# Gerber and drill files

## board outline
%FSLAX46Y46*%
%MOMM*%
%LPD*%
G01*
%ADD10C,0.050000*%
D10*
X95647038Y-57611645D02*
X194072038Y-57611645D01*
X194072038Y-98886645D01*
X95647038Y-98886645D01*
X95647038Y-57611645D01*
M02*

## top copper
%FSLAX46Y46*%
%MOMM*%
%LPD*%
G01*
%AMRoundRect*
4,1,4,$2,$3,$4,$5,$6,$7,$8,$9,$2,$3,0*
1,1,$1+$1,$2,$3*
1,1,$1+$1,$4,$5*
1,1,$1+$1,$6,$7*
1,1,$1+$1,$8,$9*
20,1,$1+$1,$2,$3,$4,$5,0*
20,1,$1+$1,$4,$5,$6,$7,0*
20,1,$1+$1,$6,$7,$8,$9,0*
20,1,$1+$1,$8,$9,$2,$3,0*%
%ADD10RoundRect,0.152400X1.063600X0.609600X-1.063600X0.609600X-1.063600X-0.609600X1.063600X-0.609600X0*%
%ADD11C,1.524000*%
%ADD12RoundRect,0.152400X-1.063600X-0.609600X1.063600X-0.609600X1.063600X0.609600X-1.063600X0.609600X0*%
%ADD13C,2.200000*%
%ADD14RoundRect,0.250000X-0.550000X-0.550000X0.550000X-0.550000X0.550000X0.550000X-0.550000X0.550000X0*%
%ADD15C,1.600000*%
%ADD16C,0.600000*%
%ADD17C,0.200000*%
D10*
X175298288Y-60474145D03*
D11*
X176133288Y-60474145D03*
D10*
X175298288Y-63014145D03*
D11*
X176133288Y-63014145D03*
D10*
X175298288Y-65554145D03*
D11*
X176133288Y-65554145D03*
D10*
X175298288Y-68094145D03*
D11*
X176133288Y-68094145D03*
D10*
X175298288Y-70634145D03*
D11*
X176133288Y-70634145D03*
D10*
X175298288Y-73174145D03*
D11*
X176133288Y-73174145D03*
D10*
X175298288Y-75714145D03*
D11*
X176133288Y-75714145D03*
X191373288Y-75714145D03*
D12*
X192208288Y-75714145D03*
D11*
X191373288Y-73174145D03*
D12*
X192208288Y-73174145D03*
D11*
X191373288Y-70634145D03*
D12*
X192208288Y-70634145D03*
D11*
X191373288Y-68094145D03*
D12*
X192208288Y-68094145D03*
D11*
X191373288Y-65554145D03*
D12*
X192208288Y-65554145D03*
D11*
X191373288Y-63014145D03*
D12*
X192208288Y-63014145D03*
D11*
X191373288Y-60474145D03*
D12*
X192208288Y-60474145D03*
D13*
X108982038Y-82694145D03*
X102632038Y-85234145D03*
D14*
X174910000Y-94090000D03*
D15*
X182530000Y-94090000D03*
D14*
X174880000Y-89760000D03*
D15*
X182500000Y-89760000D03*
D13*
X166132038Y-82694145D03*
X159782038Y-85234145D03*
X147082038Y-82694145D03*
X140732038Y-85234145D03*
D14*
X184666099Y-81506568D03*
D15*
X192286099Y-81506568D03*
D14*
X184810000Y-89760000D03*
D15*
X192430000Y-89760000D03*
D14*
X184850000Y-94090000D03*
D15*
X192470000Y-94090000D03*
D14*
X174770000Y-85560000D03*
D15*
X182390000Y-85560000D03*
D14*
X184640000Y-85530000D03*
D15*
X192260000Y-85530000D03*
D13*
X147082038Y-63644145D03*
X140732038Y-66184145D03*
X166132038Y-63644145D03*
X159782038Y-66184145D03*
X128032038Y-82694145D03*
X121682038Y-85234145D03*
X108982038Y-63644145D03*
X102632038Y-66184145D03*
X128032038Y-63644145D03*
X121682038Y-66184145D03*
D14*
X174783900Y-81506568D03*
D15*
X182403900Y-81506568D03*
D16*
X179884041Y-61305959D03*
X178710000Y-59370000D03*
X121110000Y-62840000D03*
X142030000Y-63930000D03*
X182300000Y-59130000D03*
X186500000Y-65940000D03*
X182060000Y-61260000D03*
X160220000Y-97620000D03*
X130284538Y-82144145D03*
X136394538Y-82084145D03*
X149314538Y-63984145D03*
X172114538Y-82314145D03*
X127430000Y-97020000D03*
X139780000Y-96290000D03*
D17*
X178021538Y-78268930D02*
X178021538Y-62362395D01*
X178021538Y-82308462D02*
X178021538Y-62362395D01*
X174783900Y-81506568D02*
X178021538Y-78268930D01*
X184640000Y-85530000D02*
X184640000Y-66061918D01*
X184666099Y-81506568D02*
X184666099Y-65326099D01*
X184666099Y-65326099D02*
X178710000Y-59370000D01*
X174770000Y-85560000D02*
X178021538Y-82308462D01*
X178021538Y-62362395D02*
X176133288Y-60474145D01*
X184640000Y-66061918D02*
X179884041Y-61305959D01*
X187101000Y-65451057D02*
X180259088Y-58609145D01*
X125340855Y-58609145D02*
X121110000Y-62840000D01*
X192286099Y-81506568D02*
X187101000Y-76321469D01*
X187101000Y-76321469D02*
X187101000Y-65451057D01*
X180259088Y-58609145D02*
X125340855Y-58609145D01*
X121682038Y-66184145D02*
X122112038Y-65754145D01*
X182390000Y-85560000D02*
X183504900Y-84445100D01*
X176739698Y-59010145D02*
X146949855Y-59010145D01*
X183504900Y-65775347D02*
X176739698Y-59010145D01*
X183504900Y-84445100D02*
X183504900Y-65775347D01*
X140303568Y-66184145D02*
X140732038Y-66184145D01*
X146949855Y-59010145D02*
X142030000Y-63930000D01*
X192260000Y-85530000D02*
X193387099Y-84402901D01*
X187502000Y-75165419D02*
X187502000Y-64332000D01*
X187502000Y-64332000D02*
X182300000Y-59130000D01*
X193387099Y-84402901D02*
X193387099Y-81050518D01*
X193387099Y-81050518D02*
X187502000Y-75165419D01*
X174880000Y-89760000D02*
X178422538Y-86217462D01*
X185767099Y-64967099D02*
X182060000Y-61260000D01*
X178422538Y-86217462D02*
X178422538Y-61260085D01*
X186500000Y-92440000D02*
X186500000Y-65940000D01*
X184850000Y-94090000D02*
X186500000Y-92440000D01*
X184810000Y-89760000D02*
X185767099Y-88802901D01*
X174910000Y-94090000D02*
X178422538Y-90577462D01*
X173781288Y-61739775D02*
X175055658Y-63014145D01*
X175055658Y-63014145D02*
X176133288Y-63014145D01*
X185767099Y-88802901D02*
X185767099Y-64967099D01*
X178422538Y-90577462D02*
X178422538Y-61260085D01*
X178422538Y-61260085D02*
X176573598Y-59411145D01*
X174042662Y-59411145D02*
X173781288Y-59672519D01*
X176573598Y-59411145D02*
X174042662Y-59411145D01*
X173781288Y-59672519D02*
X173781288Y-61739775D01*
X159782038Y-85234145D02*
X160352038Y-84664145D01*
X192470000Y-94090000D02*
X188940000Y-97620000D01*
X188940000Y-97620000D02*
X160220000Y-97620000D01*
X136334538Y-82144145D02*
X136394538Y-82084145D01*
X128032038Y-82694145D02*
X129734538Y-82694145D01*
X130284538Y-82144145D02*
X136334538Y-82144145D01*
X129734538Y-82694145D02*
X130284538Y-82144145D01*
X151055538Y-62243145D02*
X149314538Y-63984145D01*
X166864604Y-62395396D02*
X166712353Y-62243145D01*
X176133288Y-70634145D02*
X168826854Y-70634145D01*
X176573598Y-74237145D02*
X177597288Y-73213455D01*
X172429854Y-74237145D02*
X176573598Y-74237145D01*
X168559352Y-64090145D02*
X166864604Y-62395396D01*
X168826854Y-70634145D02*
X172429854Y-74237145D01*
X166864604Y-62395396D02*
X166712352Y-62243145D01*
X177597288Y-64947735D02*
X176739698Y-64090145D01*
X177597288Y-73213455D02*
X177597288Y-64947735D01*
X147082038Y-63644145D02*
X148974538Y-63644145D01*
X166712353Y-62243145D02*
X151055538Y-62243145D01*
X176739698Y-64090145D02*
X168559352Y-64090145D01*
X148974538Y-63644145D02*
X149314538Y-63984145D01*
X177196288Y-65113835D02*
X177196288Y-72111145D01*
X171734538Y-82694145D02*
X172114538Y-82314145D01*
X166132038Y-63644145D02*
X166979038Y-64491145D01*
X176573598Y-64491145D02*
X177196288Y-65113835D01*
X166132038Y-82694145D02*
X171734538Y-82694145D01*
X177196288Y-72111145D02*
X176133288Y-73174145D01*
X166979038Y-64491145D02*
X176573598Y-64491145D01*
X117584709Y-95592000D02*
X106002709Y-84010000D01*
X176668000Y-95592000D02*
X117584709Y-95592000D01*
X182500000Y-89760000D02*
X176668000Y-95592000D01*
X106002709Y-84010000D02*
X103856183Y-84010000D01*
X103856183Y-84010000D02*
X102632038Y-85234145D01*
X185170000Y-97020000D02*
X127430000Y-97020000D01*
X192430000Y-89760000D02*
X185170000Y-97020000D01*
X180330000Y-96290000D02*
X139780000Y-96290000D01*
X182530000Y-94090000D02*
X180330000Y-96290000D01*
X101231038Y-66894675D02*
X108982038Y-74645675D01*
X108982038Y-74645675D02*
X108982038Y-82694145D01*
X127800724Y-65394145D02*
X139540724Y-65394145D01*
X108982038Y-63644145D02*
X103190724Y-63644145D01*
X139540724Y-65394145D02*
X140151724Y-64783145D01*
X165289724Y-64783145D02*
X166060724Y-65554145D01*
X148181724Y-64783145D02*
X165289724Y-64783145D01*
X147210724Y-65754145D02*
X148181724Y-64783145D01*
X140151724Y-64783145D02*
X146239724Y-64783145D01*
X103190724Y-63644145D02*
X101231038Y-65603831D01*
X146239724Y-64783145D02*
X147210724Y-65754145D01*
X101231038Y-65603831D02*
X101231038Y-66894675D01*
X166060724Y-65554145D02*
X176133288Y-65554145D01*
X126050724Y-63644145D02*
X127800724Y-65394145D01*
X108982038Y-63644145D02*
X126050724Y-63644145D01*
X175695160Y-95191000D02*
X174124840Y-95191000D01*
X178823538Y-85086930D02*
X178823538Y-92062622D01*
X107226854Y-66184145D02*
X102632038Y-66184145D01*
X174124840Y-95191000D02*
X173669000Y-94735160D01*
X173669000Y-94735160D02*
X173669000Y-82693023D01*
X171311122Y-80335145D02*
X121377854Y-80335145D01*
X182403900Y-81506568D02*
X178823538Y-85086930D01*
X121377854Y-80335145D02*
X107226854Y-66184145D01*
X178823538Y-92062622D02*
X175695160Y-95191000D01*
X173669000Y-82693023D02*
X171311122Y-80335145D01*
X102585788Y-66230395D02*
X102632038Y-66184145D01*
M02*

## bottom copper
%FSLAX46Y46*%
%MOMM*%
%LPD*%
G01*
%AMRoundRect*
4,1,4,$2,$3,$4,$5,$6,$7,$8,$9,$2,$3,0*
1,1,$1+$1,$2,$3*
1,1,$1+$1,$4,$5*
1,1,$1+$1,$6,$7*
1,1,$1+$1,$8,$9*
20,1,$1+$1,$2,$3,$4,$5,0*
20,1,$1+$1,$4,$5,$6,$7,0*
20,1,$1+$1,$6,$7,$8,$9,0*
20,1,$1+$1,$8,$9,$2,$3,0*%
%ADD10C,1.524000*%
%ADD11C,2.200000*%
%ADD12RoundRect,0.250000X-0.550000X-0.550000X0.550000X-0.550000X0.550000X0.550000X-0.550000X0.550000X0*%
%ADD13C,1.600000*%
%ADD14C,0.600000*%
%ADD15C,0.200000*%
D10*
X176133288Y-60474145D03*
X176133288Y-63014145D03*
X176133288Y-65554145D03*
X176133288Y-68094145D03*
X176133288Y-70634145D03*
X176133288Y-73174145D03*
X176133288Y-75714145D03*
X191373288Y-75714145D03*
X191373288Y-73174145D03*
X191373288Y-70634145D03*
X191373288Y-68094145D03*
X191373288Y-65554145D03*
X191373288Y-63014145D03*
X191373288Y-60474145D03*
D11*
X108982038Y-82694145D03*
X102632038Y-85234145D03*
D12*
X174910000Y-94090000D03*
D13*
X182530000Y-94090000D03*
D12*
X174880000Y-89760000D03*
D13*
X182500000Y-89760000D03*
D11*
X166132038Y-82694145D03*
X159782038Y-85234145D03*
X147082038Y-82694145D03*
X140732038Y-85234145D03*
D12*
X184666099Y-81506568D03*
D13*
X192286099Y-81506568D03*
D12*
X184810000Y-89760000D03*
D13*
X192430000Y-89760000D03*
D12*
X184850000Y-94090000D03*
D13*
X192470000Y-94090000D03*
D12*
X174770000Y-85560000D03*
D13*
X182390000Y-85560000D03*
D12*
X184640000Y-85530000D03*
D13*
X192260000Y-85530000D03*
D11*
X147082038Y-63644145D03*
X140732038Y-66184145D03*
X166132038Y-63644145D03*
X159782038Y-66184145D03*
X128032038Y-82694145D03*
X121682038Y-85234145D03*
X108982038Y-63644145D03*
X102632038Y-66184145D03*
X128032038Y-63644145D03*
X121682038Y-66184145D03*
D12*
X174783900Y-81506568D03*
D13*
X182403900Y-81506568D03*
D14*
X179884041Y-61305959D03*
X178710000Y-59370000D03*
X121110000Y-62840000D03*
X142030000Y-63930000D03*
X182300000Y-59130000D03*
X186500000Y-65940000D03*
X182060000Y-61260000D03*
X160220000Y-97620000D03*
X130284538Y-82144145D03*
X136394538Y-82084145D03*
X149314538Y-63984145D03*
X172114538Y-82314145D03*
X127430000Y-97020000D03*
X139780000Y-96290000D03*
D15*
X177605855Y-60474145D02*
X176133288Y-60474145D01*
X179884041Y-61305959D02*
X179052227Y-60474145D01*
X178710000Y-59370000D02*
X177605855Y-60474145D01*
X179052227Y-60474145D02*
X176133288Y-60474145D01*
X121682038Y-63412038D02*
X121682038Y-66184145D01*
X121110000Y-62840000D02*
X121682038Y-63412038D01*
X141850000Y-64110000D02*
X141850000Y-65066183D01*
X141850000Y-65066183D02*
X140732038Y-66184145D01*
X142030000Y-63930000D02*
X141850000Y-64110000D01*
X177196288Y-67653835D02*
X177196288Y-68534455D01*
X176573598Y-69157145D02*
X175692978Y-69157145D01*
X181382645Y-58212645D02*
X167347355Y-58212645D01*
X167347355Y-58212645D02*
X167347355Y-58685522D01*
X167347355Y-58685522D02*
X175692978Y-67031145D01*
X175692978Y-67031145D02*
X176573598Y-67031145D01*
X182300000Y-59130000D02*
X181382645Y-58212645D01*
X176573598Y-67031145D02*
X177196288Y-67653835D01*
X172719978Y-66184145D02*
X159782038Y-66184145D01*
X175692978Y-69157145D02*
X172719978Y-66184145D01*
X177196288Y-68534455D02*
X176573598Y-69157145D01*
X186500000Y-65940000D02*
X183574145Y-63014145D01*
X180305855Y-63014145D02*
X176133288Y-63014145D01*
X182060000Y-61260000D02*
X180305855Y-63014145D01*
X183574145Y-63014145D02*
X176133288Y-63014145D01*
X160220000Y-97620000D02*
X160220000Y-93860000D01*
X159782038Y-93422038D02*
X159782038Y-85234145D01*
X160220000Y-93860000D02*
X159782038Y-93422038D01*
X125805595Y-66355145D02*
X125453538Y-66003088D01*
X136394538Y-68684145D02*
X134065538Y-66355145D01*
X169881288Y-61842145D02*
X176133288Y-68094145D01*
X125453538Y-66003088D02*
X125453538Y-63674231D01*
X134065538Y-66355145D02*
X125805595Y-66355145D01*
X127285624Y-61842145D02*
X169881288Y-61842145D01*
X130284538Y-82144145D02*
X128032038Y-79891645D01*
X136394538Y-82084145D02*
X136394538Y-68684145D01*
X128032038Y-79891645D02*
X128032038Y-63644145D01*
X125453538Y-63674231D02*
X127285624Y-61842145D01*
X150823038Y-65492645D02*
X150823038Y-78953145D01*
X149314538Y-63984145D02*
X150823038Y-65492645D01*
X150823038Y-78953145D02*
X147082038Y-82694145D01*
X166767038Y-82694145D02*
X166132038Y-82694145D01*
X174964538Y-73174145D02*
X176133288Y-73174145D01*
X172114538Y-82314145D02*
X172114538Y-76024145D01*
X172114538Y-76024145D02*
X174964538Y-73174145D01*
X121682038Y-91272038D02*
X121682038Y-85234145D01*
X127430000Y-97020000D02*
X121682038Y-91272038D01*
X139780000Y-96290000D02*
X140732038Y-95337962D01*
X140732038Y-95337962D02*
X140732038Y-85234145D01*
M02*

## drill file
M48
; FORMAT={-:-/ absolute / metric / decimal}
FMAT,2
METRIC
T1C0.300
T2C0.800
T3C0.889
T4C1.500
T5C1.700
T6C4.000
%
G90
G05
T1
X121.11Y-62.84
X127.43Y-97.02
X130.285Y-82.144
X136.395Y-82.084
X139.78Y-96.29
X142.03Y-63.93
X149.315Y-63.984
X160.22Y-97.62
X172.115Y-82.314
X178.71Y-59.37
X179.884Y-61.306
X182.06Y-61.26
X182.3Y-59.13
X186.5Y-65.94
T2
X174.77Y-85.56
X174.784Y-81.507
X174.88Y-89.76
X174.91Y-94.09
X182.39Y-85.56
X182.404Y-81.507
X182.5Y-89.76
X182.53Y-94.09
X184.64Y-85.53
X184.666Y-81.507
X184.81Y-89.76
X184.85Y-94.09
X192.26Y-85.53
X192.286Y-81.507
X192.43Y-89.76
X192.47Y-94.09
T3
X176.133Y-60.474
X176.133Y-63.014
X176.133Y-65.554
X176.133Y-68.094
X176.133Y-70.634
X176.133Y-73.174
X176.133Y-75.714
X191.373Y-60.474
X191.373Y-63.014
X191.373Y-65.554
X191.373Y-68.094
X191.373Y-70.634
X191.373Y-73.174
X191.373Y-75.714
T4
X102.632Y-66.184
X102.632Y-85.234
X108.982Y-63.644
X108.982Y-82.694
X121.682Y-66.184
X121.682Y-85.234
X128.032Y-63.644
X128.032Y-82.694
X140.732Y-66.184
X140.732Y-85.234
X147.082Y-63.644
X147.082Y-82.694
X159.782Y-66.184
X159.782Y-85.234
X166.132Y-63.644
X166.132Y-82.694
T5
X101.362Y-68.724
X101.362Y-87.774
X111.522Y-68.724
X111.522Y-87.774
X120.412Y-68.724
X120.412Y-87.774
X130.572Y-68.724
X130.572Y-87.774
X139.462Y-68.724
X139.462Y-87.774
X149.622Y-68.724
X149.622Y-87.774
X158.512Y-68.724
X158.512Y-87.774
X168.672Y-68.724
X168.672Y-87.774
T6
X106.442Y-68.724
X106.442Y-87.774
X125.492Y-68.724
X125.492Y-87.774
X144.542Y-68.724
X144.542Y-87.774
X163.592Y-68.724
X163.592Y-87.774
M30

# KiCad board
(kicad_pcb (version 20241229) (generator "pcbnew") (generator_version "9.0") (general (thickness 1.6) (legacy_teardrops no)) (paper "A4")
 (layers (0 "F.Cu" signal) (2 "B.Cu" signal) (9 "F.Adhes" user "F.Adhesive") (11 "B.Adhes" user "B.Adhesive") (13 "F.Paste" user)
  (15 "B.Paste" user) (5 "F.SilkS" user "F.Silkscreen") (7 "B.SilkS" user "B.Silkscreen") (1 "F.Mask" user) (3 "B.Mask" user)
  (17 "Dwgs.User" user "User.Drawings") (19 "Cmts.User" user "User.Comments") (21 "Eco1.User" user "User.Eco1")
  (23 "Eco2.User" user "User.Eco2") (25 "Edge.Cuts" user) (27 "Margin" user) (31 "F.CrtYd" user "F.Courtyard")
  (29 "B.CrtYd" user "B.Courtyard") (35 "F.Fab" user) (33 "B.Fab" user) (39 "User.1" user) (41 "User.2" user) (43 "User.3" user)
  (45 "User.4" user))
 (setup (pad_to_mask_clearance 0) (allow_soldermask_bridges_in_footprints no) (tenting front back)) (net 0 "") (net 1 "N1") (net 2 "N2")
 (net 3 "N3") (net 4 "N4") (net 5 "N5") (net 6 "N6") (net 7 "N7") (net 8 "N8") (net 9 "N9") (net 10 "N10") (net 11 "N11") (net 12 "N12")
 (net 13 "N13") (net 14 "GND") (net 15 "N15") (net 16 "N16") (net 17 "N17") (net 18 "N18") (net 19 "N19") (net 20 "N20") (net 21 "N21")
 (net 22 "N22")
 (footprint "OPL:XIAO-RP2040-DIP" (layer "F.Cu") (at 183.753288 68.094145)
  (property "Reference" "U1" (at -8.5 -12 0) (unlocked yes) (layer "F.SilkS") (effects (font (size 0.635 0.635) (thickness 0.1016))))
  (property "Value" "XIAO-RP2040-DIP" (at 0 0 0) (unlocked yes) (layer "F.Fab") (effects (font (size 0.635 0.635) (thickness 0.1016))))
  (pad "1" smd roundrect (at -8.455 -7.62 180) (size 2.432 1.524) (layers "F.Cu" "F.Mask") (roundrect_rratio 0.1) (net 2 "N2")
   (thermal_bridge_angle 45))
  (pad "1" thru_hole circle (at -7.62 -7.62 180) (size 1.524 1.524) (drill 0.889) (layers "*.Cu" "*.Mask") (remove_unused_layers no)
   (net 2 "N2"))
  (pad "2" smd roundrect (at -8.455 -5.08 180) (size 2.432 1.524) (layers "F.Cu" "F.Mask") (roundrect_rratio 0.1) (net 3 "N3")
   (thermal_bridge_angle 45))
  (pad "2" thru_hole circle (at -7.62 -5.08 180) (size 1.524 1.524) (drill 0.889) (layers "*.Cu" "*.Mask") (remove_unused_layers no)
   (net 3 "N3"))
  (pad "3" smd roundrect (at -8.455 -2.54 180) (size 2.432 1.524) (layers "F.Cu" "F.Mask") (roundrect_rratio 0.1) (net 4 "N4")
   (thermal_bridge_angle 45))
  (pad "3" thru_hole circle (at -7.62 -2.54 180) (size 1.524 1.524) (drill 0.889) (layers "*.Cu" "*.Mask") (remove_unused_layers no)
   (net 4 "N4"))
  (pad "4" smd roundrect (at -8.455 0 180) (size 2.432 1.524) (layers "F.Cu" "F.Mask") (roundrect_rratio 0.1) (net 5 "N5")
   (thermal_bridge_angle 45))
  (pad "4" thru_hole circle (at -7.62 0 180) (size 1.524 1.524) (drill 0.889) (layers "*.Cu" "*.Mask") (remove_unused_layers no)
   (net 5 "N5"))
  (pad "5" smd roundrect (at -8.455 2.54 180) (size 2.432 1.524) (layers "F.Cu" "F.Mask") (roundrect_rratio 0.1) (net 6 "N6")
   (thermal_bridge_angle 45))
  (pad "5" thru_hole circle (at -7.62 2.54 180) (size 1.524 1.524) (drill 0.889) (layers "*.Cu" "*.Mask") (remove_unused_layers no)
   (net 6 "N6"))
  (pad "6" smd roundrect (at -8.455 5.08 180) (size 2.432 1.524) (layers "F.Cu" "F.Mask") (roundrect_rratio 0.1) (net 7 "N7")
   (thermal_bridge_angle 45))
  (pad "6" thru_hole circle (at -7.62 5.08 180) (size 1.524 1.524) (drill 0.889) (layers "*.Cu" "*.Mask") (remove_unused_layers no)
   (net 7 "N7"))
  (pad "7" smd roundrect (at -8.455 7.62 180) (size 2.432 1.524) (layers "F.Cu" "F.Mask") (roundrect_rratio 0.1) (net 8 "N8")
   (thermal_bridge_angle 45))
  (pad "7" thru_hole circle (at -7.62 7.62 180) (size 1.524 1.524) (drill 0.889) (layers "*.Cu" "*.Mask") (remove_unused_layers no)
   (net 8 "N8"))
  (pad "8" thru_hole circle (at 7.62 7.62) (size 1.524 1.524) (drill 0.889) (layers "*.Cu" "*.Mask") (remove_unused_layers no) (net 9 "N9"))
  (pad "8" smd roundrect (at 8.455 7.62) (size 2.432 1.524) (layers "F.Cu" "F.Mask") (roundrect_rratio 0.1) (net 9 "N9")
   (thermal_bridge_angle 45))
  (pad "9" thru_hole circle (at 7.62 5.08) (size 1.524 1.524) (drill 0.889) (layers "*.Cu" "*.Mask") (remove_unused_layers no)
   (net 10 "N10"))
  (pad "9" smd roundrect (at 8.455 5.08) (size 2.432 1.524) (layers "F.Cu" "F.Mask") (roundrect_rratio 0.1) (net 10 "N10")
   (thermal_bridge_angle 45))
  (pad "10" thru_hole circle (at 7.62 2.54) (size 1.524 1.524) (drill 0.889) (layers "*.Cu" "*.Mask") (remove_unused_layers no)
   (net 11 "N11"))
  (pad "10" smd roundrect (at 8.455 2.54) (size 2.432 1.524) (layers "F.Cu" "F.Mask") (roundrect_rratio 0.1) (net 11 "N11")
   (thermal_bridge_angle 45))
  (pad "11" thru_hole circle (at 7.62 0) (size 1.524 1.524) (drill 0.889) (layers "*.Cu" "*.Mask") (remove_unused_layers no) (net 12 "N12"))
  (pad "11" smd roundrect (at 8.455 0) (size 2.432 1.524) (layers "F.Cu" "F.Mask") (roundrect_rratio 0.1) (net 12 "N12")
   (thermal_bridge_angle 45))
  (pad "12" thru_hole circle (at 7.62 -2.54) (size 1.524 1.524) (drill 0.889) (layers "*.Cu" "*.Mask") (remove_unused_layers no)
   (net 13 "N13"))
  (pad "12" smd roundrect (at 8.455 -2.54) (size 2.432 1.524) (layers "F.Cu" "F.Mask") (roundrect_rratio 0.1) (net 13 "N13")
   (thermal_bridge_angle 45))
  (pad "13" thru_hole circle (at 7.62 -5.08) (size 1.524 1.524) (drill 0.889) (layers "*.Cu" "*.Mask") (remove_unused_layers no)
   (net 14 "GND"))
  (pad "13" smd roundrect (at 8.455 -5.08) (size 2.432 1.524) (layers "F.Cu" "F.Mask") (roundrect_rratio 0.1) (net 14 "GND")
   (thermal_bridge_angle 45))
  (pad "14" thru_hole circle (at 7.62 -7.62) (size 1.524 1.524) (drill 0.889) (layers "*.Cu" "*.Mask") (remove_unused_layers no)
   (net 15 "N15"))
  (pad "14" smd roundrect (at 8.455 -7.62) (size 2.432 1.524) (layers "F.Cu" "F.Mask") (roundrect_rratio 0.1) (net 15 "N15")
   (thermal_bridge_angle 45)))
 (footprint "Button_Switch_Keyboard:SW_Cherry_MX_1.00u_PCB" (layer "F.Cu") (at 108.982038 82.694145)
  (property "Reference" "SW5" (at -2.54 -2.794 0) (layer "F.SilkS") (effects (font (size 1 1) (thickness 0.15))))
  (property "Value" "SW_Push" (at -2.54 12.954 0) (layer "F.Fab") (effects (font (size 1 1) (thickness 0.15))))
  (pad "" np_thru_hole circle (at -7.62 5.08) (size 1.7 1.7) (drill 1.7) (layers "*.Cu" "*.Mask"))
  (pad "" np_thru_hole circle (at -2.54 5.08) (size 4 4) (drill 4) (layers "*.Cu" "*.Mask"))
  (pad "" np_thru_hole circle (at 2.54 5.08) (size 1.7 1.7) (drill 1.7) (layers "*.Cu" "*.Mask"))
  (pad "1" thru_hole circle (at 0 0) (size 2.2 2.2) (drill 1.5) (layers "*.Cu" "*.Mask") (remove_unused_layers no) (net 4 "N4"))
  (pad "2" thru_hole circle (at -6.35 2.54) (size 2.2 2.2) (drill 1.5) (layers "*.Cu" "*.Mask") (remove_unused_layers no) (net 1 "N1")))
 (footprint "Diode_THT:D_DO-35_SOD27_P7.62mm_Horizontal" (layer "F.Cu") (at 174.91 94.09)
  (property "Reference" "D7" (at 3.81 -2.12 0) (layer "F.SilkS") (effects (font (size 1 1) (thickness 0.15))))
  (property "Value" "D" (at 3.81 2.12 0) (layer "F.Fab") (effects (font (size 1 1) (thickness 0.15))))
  (pad "1" thru_hole roundrect (at 0 0) (size 1.6 1.6) (drill 0.8) (layers "*.Cu" "*.Mask") (remove_unused_layers no)
   (roundrect_rratio 0.15625) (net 3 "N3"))
  (pad "2" thru_hole circle (at 7.62 0) (size 1.6 1.6) (drill 0.8) (layers "*.Cu" "*.Mask") (remove_unused_layers no) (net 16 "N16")))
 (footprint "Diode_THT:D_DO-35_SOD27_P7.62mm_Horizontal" (layer "F.Cu") (at 174.88 89.76)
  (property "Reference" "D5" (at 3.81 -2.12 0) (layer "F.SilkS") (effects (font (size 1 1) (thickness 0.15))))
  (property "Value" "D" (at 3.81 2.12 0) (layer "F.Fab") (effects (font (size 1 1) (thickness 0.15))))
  (pad "1" thru_hole roundrect (at 0 0) (size 1.6 1.6) (drill 0.8) (layers "*.Cu" "*.Mask") (remove_unused_layers no)
   (roundrect_rratio 0.15625) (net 3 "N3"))
  (pad "2" thru_hole circle (at 7.62 0) (size 1.6 1.6) (drill 0.8) (layers "*.Cu" "*.Mask") (remove_unused_layers no) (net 1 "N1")))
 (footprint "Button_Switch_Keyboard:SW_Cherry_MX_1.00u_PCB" (layer "F.Cu") (at 166.132038 82.694145)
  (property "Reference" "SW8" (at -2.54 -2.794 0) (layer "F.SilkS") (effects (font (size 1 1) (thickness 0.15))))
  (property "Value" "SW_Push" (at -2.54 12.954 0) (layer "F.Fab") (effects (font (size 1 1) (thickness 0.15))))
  (pad "" np_thru_hole circle (at -7.62 5.08) (size 1.7 1.7) (drill 1.7) (layers "*.Cu" "*.Mask"))
  (pad "" np_thru_hole circle (at -2.54 5.08) (size 4 4) (drill 4) (layers "*.Cu" "*.Mask"))
  (pad "" np_thru_hole circle (at 2.54 5.08) (size 1.7 1.7) (drill 1.7) (layers "*.Cu" "*.Mask"))
  (pad "1" thru_hole circle (at 0 0) (size 2.2 2.2) (drill 1.5) (layers "*.Cu" "*.Mask") (remove_unused_layers no) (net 7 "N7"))
  (pad "2" thru_hole circle (at -6.35 2.54) (size 2.2 2.2) (drill 1.5) (layers "*.Cu" "*.Mask") (remove_unused_layers no) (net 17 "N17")))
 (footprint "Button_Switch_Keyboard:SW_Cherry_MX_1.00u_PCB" (layer "F.Cu") (at 147.082038 82.694145)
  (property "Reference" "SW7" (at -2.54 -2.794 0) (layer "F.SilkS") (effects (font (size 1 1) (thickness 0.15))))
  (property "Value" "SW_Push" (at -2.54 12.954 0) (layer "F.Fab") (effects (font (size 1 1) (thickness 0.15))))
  (pad "" np_thru_hole circle (at -7.62 5.08) (size 1.7 1.7) (drill 1.7) (layers "*.Cu" "*.Mask"))
  (pad "" np_thru_hole circle (at -2.54 5.08) (size 4 4) (drill 4) (layers "*.Cu" "*.Mask"))
  (pad "" np_thru_hole circle (at 2.54 5.08) (size 1.7 1.7) (drill 1.7) (layers "*.Cu" "*.Mask"))
  (pad "1" thru_hole circle (at 0 0) (size 2.2 2.2) (drill 1.5) (layers "*.Cu" "*.Mask") (remove_unused_layers no) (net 6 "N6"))
  (pad "2" thru_hole circle (at -6.35 2.54) (size 2.2 2.2) (drill 1.5) (layers "*.Cu" "*.Mask") (remove_unused_layers no) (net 16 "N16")))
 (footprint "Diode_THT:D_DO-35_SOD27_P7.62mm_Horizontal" (layer "F.Cu") (at 184.666099 81.506568)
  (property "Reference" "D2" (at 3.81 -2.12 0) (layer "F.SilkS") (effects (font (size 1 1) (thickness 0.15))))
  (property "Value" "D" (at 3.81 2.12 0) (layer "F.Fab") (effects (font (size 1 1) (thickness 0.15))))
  (pad "1" thru_hole roundrect (at 0 0) (size 1.6 1.6) (drill 0.8) (layers "*.Cu" "*.Mask") (remove_unused_layers no)
   (roundrect_rratio 0.15625) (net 2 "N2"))
  (pad "2" thru_hole circle (at 7.62 0) (size 1.6 1.6) (drill 0.8) (layers "*.Cu" "*.Mask") (remove_unused_layers no) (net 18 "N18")))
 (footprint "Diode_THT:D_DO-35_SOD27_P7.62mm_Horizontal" (layer "F.Cu") (at 184.81 89.76)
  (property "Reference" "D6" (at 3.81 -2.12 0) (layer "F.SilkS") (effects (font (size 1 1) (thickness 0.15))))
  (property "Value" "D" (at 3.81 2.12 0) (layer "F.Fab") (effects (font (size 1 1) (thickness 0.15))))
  (pad "1" thru_hole roundrect (at 0 0) (size 1.6 1.6) (drill 0.8) (layers "*.Cu" "*.Mask") (remove_unused_layers no)
   (roundrect_rratio 0.15625) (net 3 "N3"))
  (pad "2" thru_hole circle (at 7.62 0) (size 1.6 1.6) (drill 0.8) (layers "*.Cu" "*.Mask") (remove_unused_layers no) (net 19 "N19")))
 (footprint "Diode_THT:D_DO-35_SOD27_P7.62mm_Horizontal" (layer "F.Cu") (at 184.85 94.09)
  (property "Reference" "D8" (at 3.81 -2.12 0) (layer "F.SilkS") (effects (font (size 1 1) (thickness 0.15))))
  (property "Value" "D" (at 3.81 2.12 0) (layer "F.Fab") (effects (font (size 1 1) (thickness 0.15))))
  (pad "1" thru_hole roundrect (at 0 0) (size 1.6 1.6) (drill 0.8) (layers "*.Cu" "*.Mask") (remove_unused_layers no)
   (roundrect_rratio 0.15625) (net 3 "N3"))
  (pad "2" thru_hole circle (at 7.62 0) (size 1.6 1.6) (drill 0.8) (layers "*.Cu" "*.Mask") (remove_unused_layers no) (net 17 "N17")))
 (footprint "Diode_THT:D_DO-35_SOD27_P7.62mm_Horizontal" (layer "F.Cu") (at 174.77 85.56)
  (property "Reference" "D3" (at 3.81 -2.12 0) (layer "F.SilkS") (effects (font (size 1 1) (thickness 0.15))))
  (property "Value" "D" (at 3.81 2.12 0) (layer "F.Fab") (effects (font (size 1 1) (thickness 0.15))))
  (pad "1" thru_hole roundrect (at 0 0) (size 1.6 1.6) (drill 0.8) (layers "*.Cu" "*.Mask") (remove_unused_layers no)
   (roundrect_rratio 0.15625) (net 2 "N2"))
  (pad "2" thru_hole circle (at 7.62 0) (size 1.6 1.6) (drill 0.8) (layers "*.Cu" "*.Mask") (remove_unused_layers no) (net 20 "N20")))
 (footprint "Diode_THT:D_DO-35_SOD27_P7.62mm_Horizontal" (layer "F.Cu") (at 184.64 85.53)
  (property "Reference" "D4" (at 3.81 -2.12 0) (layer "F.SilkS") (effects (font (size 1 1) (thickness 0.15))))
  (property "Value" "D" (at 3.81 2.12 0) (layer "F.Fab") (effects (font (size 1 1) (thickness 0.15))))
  (pad "1" thru_hole roundrect (at 0 0) (size 1.6 1.6) (drill 0.8) (layers "*.Cu" "*.Mask") (remove_unused_layers no)
   (roundrect_rratio 0.15625) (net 2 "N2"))
  (pad "2" thru_hole circle (at 7.62 0) (size 1.6 1.6) (drill 0.8) (layers "*.Cu" "*.Mask") (remove_unused_layers no) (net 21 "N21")))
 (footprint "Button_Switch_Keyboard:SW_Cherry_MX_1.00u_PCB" (layer "F.Cu") (at 147.082038 63.644145)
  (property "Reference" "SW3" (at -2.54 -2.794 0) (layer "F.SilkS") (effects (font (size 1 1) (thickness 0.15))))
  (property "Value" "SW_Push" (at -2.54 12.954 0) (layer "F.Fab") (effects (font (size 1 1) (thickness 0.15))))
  (pad "" np_thru_hole circle (at -7.62 5.08) (size 1.7 1.7) (drill 1.7) (layers "*.Cu" "*.Mask"))
  (pad "" np_thru_hole circle (at -2.54 5.08) (size 4 4) (drill 4) (layers "*.Cu" "*.Mask"))
  (pad "" np_thru_hole circle (at 2.54 5.08) (size 1.7 1.7) (drill 1.7) (layers "*.Cu" "*.Mask"))
  (pad "1" thru_hole circle (at 0 0) (size 2.2 2.2) (drill 1.5) (layers "*.Cu" "*.Mask") (remove_unused_layers no) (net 6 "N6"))
  (pad "2" thru_hole circle (at -6.35 2.54) (size 2.2 2.2) (drill 1.5) (layers "*.Cu" "*.Mask") (remove_unused_layers no) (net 20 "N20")))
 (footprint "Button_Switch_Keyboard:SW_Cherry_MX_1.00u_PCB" (layer "F.Cu") (at 166.132038 63.644145)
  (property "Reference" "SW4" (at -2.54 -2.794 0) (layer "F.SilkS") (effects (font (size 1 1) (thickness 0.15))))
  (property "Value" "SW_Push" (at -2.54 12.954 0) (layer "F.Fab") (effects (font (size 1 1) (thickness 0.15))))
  (pad "" np_thru_hole circle (at -7.62 5.08) (size 1.7 1.7) (drill 1.7) (layers "*.Cu" "*.Mask"))
  (pad "" np_thru_hole circle (at -2.54 5.08) (size 4 4) (drill 4) (layers "*.Cu" "*.Mask"))
  (pad "" np_thru_hole circle (at 2.54 5.08) (size 1.7 1.7) (drill 1.7) (layers "*.Cu" "*.Mask"))
  (pad "1" thru_hole circle (at 0 0) (size 2.2 2.2) (drill 1.5) (layers "*.Cu" "*.Mask") (remove_unused_layers no) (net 7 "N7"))
  (pad "2" thru_hole circle (at -6.35 2.54) (size 2.2 2.2) (drill 1.5) (layers "*.Cu" "*.Mask") (remove_unused_layers no) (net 21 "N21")))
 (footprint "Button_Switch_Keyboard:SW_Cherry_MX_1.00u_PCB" (layer "F.Cu") (at 128.032038 82.694145)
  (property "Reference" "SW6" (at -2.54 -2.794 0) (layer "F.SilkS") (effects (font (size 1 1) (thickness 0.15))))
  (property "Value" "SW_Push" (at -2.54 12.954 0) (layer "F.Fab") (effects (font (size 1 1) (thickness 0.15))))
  (pad "" np_thru_hole circle (at -7.62 5.08) (size 1.7 1.7) (drill 1.7) (layers "*.Cu" "*.Mask"))
  (pad "" np_thru_hole circle (at -2.54 5.08) (size 4 4) (drill 4) (layers "*.Cu" "*.Mask"))
  (pad "" np_thru_hole circle (at 2.54 5.08) (size 1.7 1.7) (drill 1.7) (layers "*.Cu" "*.Mask"))
  (pad "1" thru_hole circle (at 0 0) (size 2.2 2.2) (drill 1.5) (layers "*.Cu" "*.Mask") (remove_unused_layers no) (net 5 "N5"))
  (pad "2" thru_hole circle (at -6.35 2.54) (size 2.2 2.2) (drill 1.5) (layers "*.Cu" "*.Mask") (remove_unused_layers no) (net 19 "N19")))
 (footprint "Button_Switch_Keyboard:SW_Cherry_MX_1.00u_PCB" (layer "F.Cu") (at 108.982038 63.644145)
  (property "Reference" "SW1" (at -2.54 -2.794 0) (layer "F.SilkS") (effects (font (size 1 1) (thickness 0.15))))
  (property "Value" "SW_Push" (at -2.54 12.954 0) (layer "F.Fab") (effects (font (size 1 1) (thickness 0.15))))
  (pad "" np_thru_hole circle (at -7.62 5.08) (size 1.7 1.7) (drill 1.7) (layers "*.Cu" "*.Mask"))
  (pad "" np_thru_hole circle (at -2.54 5.08) (size 4 4) (drill 4) (layers "*.Cu" "*.Mask"))
  (pad "" np_thru_hole circle (at 2.54 5.08) (size 1.7 1.7) (drill 1.7) (layers "*.Cu" "*.Mask"))
  (pad "1" thru_hole circle (at 0 0) (size 2.2 2.2) (drill 1.5) (layers "*.Cu" "*.Mask") (remove_unused_layers no) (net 4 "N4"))
  (pad "2" thru_hole circle (at -6.35 2.54) (size 2.2 2.2) (drill 1.5) (layers "*.Cu" "*.Mask") (remove_unused_layers no) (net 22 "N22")))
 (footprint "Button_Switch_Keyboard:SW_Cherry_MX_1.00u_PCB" (layer "F.Cu") (at 128.032038 63.644145)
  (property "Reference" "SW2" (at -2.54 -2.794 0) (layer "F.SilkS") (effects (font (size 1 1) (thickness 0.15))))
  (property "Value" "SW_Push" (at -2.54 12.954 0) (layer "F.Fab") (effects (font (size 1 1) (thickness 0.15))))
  (pad "" np_thru_hole circle (at -7.62 5.08) (size 1.7 1.7) (drill 1.7) (layers "*.Cu" "*.Mask"))
  (pad "" np_thru_hole circle (at -2.54 5.08) (size 4 4) (drill 4) (layers "*.Cu" "*.Mask"))
  (pad "" np_thru_hole circle (at 2.54 5.08) (size 1.7 1.7) (drill 1.7) (layers "*.Cu" "*.Mask"))
  (pad "1" thru_hole circle (at 0 0) (size 2.2 2.2) (drill 1.5) (layers "*.Cu" "*.Mask") (remove_unused_layers no) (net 5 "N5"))
  (pad "2" thru_hole circle (at -6.35 2.54) (size 2.2 2.2) (drill 1.5) (layers "*.Cu" "*.Mask") (remove_unused_layers no) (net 18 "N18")))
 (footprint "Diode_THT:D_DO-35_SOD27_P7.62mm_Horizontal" (layer "F.Cu") (at 174.7839 81.506568)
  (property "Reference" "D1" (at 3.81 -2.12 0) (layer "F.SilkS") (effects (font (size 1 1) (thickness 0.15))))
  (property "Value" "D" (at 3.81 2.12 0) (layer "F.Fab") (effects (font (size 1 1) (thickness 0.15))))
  (pad "1" thru_hole roundrect (at 0 0) (size 1.6 1.6) (drill 0.8) (layers "*.Cu" "*.Mask") (remove_unused_layers no)
   (roundrect_rratio 0.15625) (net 2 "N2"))
  (pad "2" thru_hole circle (at 7.62 0) (size 1.6 1.6) (drill 0.8) (layers "*.Cu" "*.Mask") (remove_unused_layers no) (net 22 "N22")))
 (gr_rect (start 95.647038 57.611645) (end 194.072038 98.886645) (stroke (width 0.05) (type default)) (fill no) (layer "Edge.Cuts"))
 (segment (start 178.021538 78.26893) (end 178.021538 62.362395) (width 0.2) (layer "F.Cu") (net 2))
 (segment (start 178.021538 82.308462) (end 178.021538 62.362395) (width 0.2) (layer "F.Cu") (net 2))
 (segment (start 174.7839 81.506568) (end 178.021538 78.26893) (width 0.2) (layer "F.Cu") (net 2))
 (segment (start 184.64 85.53) (end 184.64 66.061918) (width 0.2) (layer "F.Cu") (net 2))
 (segment (start 184.666099 81.506568) (end 184.666099 65.326099) (width 0.2) (layer "F.Cu") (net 2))
 (segment (start 184.666099 65.326099) (end 178.71 59.37) (width 0.2) (layer "F.Cu") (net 2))
 (segment (start 174.77 85.56) (end 178.021538 82.308462) (width 0.2) (layer "F.Cu") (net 2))
 (segment (start 178.021538 62.362395) (end 176.133288 60.474145) (width 0.2) (layer "F.Cu") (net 2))
 (segment (start 184.64 66.061918) (end 179.884041 61.305959) (width 0.2) (layer "F.Cu") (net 2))
 (via (at 179.884041 61.305959) (size 0.6) (drill 0.3) (layers "F.Cu" "B.Cu") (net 2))
 (via (at 178.71 59.37) (size 0.6) (drill 0.3) (layers "F.Cu" "B.Cu") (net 2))
 (segment (start 177.605855 60.474145) (end 176.133288 60.474145) (width 0.2) (layer "B.Cu") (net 2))
 (segment (start 179.884041 61.305959) (end 179.052227 60.474145) (width 0.2) (layer "B.Cu") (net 2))
 (segment (start 178.71 59.37) (end 177.605855 60.474145) (width 0.2) (layer "B.Cu") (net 2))
 (segment (start 179.052227 60.474145) (end 176.133288 60.474145) (width 0.2) (layer "B.Cu") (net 2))
 (segment (start 187.101 65.451057) (end 180.259088 58.609145) (width 0.2) (layer "F.Cu") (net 18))
 (segment (start 125.340855 58.609145) (end 121.11 62.84) (width 0.2) (layer "F.Cu") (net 18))
 (segment (start 192.286099 81.506568) (end 187.101 76.321469) (width 0.2) (layer "F.Cu") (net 18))
 (segment (start 187.101 76.321469) (end 187.101 65.451057) (width 0.2) (layer "F.Cu") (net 18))
 (segment (start 180.259088 58.609145) (end 125.340855 58.609145) (width 0.2) (layer "F.Cu") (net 18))
 (segment (start 121.682038 66.184145) (end 122.112038 65.754145) (width 0.2) (layer "F.Cu") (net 18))
 (via (at 121.11 62.84) (size 0.6) (drill 0.3) (layers "F.Cu" "B.Cu") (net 18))
 (segment (start 121.682038 63.412038) (end 121.682038 66.184145) (width 0.2) (layer "B.Cu") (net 18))
 (segment (start 121.11 62.84) (end 121.682038 63.412038) (width 0.2) (layer "B.Cu") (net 18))
 (segment (start 182.39 85.56) (end 183.5049 84.4451) (width 0.2) (layer "F.Cu") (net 20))
 (segment (start 176.739698 59.010145) (end 146.949855 59.010145) (width 0.2) (layer "F.Cu") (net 20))
 (segment (start 183.5049 65.775347) (end 176.739698 59.010145) (width 0.2) (layer "F.Cu") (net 20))
 (segment (start 183.5049 84.4451) (end 183.5049 65.775347) (width 0.2) (layer "F.Cu") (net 20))
 (segment (start 140.303568 66.184145) (end 140.732038 66.184145) (width 0.2) (layer "F.Cu") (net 20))
 (segment (start 146.949855 59.010145) (end 142.03 63.93) (width 0.2) (layer "F.Cu") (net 20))
 (via (at 142.03 63.93) (size 0.6) (drill 0.3) (layers "F.Cu" "B.Cu") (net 20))
 (segment (start 141.85 64.11) (end 141.85 65.066183) (width 0.2) (layer "B.Cu") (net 20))
 (segment (start 141.85 65.066183) (end 140.732038 66.184145) (width 0.2) (layer "B.Cu") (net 20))
 (segment (start 142.03 63.93) (end 141.85 64.11) (width 0.2) (layer "B.Cu") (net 20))
 (segment (start 192.26 85.53) (end 193.387099 84.402901) (width 0.2) (layer "F.Cu") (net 21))
 (segment (start 187.502 75.165419) (end 187.502 64.332) (width 0.2) (layer "F.Cu") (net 21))
 (segment (start 187.502 64.332) (end 182.3 59.13) (width 0.2) (layer "F.Cu") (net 21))
 (segment (start 193.387099 84.402901) (end 193.387099 81.050518) (width 0.2) (layer "F.Cu") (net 21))
 (segment (start 193.387099 81.050518) (end 187.502 75.165419) (width 0.2) (layer "F.Cu") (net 21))
 (via (at 182.3 59.13) (size 0.6) (drill 0.3) (layers "F.Cu" "B.Cu") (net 21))
 (segment (start 177.196288 67.653835) (end 177.196288 68.534455) (width 0.2) (layer "B.Cu") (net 21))
 (segment (start 176.573598 69.157145) (end 175.692978 69.157145) (width 0.2) (layer "B.Cu") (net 21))
 (segment (start 181.382645 58.212645) (end 167.347355 58.212645) (width 0.2) (layer "B.Cu") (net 21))
 (segment (start 167.347355 58.212645) (end 167.347355 58.685522) (width 0.2) (layer "B.Cu") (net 21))
 (segment (start 167.347355 58.685522) (end 175.692978 67.031145) (width 0.2) (layer "B.Cu") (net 21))
 (segment (start 175.692978 67.031145) (end 176.573598 67.031145) (width 0.2) (layer "B.Cu") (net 21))
 (segment (start 182.3 59.13) (end 181.382645 58.212645) (width 0.2) (layer "B.Cu") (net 21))
 (segment (start 176.573598 67.031145) (end 177.196288 67.653835) (width 0.2) (layer "B.Cu") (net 21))
 (segment (start 172.719978 66.184145) (end 159.782038 66.184145) (width 0.2) (layer "B.Cu") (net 21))
 (segment (start 175.692978 69.157145) (end 172.719978 66.184145) (width 0.2) (layer "B.Cu") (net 21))
 (segment (start 177.196288 68.534455) (end 176.573598 69.157145) (width 0.2) (layer "B.Cu") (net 21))
 (segment (start 174.88 89.76) (end 178.422538 86.217462) (width 0.2) (layer "F.Cu") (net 3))
 (segment (start 185.767099 64.967099) (end 182.06 61.26) (width 0.2) (layer "F.Cu") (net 3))
 (segment (start 178.422538 86.217462) (end 178.422538 61.260085) (width 0.2) (layer "F.Cu") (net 3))
 (segment (start 186.5 92.44) (end 186.5 65.94) (width 0.2) (layer "F.Cu") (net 3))
 (segment (start 184.85 94.09) (end 186.5 92.44) (width 0.2) (layer "F.Cu") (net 3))
 (segment (start 184.81 89.76) (end 185.767099 88.802901) (width 0.2) (layer "F.Cu") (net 3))
 (segment (start 174.91 94.09) (end 178.422538 90.577462) (width 0.2) (layer "F.Cu") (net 3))
 (segment (start 173.781288 61.739775) (end 175.055658 63.014145) (width 0.2) (layer "F.Cu") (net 3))
 (segment (start 175.055658 63.014145) (end 176.133288 63.014145) (width 0.2) (layer "F.Cu") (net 3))
 (segment (start 185.767099 88.802901) (end 185.767099 64.967099) (width 0.2) (layer "F.Cu") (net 3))
 (segment (start 178.422538 90.577462) (end 178.422538 61.260085) (width 0.2) (layer "F.Cu") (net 3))
 (segment (start 178.422538 61.260085) (end 176.573598 59.411145) (width 0.2) (layer "F.Cu") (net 3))
 (segment (start 174.042662 59.411145) (end 173.781288 59.672519) (width 0.2) (layer "F.Cu") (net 3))
 (segment (start 176.573598 59.411145) (end 174.042662 59.411145) (width 0.2) (layer "F.Cu") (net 3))
 (segment (start 173.781288 59.672519) (end 173.781288 61.739775) (width 0.2) (layer "F.Cu") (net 3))
 (via (at 186.5 65.94) (size 0.6) (drill 0.3) (layers "F.Cu" "B.Cu") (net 3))
 (via (at 182.06 61.26) (size 0.6) (drill 0.3) (layers "F.Cu" "B.Cu") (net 3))
 (segment (start 186.5 65.94) (end 183.574145 63.014145) (width 0.2) (layer "B.Cu") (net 3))
 (segment (start 180.305855 63.014145) (end 176.133288 63.014145) (width 0.2) (layer "B.Cu") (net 3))
 (segment (start 182.06 61.26) (end 180.305855 63.014145) (width 0.2) (layer "B.Cu") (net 3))
 (segment (start 183.574145 63.014145) (end 176.133288 63.014145) (width 0.2) (layer "B.Cu") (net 3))
 (segment (start 159.782038 85.234145) (end 160.352038 84.664145) (width 0.2) (layer "F.Cu") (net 17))
 (segment (start 192.47 94.09) (end 188.94 97.62) (width 0.2) (layer "F.Cu") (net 17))
 (segment (start 188.94 97.62) (end 160.22 97.62) (width 0.2) (layer "F.Cu") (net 17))
 (via (at 160.22 97.62) (size 0.6) (drill 0.3) (layers "F.Cu" "B.Cu") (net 17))
 (segment (start 160.22 97.62) (end 160.22 93.86) (width 0.2) (layer "B.Cu") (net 17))
 (segment (start 159.782038 93.422038) (end 159.782038 85.234145) (width 0.2) (layer "B.Cu") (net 17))
 (segment (start 160.22 93.86) (end 159.782038 93.422038) (width 0.2) (layer "B.Cu") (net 17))
 (segment (start 136.334538 82.144145) (end 136.394538 82.084145) (width 0.2) (layer "F.Cu") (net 5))
 (segment (start 128.032038 82.694145) (end 129.734538 82.694145) (width 0.2) (layer "F.Cu") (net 5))
 (segment (start 130.284538 82.144145) (end 136.334538 82.144145) (width 0.2) (layer "F.Cu") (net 5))
 (segment (start 129.734538 82.694145) (end 130.284538 82.144145) (width 0.2) (layer "F.Cu") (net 5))
 (via (at 130.284538 82.144145) (size 0.6) (drill 0.3) (layers "F.Cu" "B.Cu") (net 5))
 (via (at 136.394538 82.084145) (size 0.6) (drill 0.3) (layers "F.Cu" "B.Cu") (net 5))
 (segment (start 125.805595 66.355145) (end 125.453538 66.003088) (width 0.2) (layer "B.Cu") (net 5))
 (segment (start 136.394538 68.684145) (end 134.065538 66.355145) (width 0.2) (layer "B.Cu") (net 5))
 (segment (start 169.881288 61.842145) (end 176.133288 68.094145) (width 0.2) (layer "B.Cu") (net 5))
 (segment (start 125.453538 66.003088) (end 125.453538 63.674231) (width 0.2) (layer "B.Cu") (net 5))
 (segment (start 134.065538 66.355145) (end 125.805595 66.355145) (width 0.2) (layer "B.Cu") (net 5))
 (segment (start 127.285624 61.842145) (end 169.881288 61.842145) (width 0.2) (layer "B.Cu") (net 5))
 (segment (start 130.284538 82.144145) (end 128.032038 79.891645) (width 0.2) (layer "B.Cu") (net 5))
 (segment (start 136.394538 82.084145) (end 136.394538 68.684145) (width 0.2) (layer "B.Cu") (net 5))
 (segment (start 128.032038 79.891645) (end 128.032038 63.644145) (width 0.2) (layer "B.Cu") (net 5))
 (segment (start 125.453538 63.674231) (end 127.285624 61.842145) (width 0.2) (layer "B.Cu") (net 5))
 (segment (start 151.055538 62.243145) (end 149.314538 63.984145) (width 0.2) (layer "F.Cu") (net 6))
 (segment (start 166.864604 62.395396) (end 166.712353 62.243145) (width 0.2) (layer "F.Cu") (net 6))
 (segment (start 176.133288 70.634145) (end 168.826854 70.634145) (width 0.2) (layer "F.Cu") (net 6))
 (segment (start 176.573598 74.237145) (end 177.597288 73.213455) (width 0.2) (layer "F.Cu") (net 6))
 (segment (start 172.429854 74.237145) (end 176.573598 74.237145) (width 0.2) (layer "F.Cu") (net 6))
 (segment (start 168.559352 64.090145) (end 166.864604 62.395396) (width 0.2) (layer "F.Cu") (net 6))
 (segment (start 168.826854 70.634145) (end 172.429854 74.237145) (width 0.2) (layer "F.Cu") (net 6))
 (segment (start 166.864604 62.395396) (end 166.712352 62.243145) (width 0.2) (layer "F.Cu") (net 6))
 (segment (start 177.597288 64.947735) (end 176.739698 64.090145) (width 0.2) (layer "F.Cu") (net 6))
 (segment (start 177.597288 73.213455) (end 177.597288 64.947735) (width 0.2) (layer "F.Cu") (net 6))
 (segment (start 147.082038 63.644145) (end 148.974538 63.644145) (width 0.2) (layer "F.Cu") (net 6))
 (segment (start 166.712353 62.243145) (end 151.055538 62.243145) (width 0.2) (layer "F.Cu") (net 6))
 (segment (start 176.739698 64.090145) (end 168.559352 64.090145) (width 0.2) (layer "F.Cu") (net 6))
 (segment (start 148.974538 63.644145) (end 149.314538 63.984145) (width 0.2) (layer "F.Cu") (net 6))
 (via (at 149.314538 63.984145) (size 0.6) (drill 0.3) (layers "F.Cu" "B.Cu") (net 6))
 (segment (start 150.823038 65.492645) (end 150.823038 78.953145) (width 0.2) (layer "B.Cu") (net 6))
 (segment (start 149.314538 63.984145) (end 150.823038 65.492645) (width 0.2) (layer "B.Cu") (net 6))
 (segment (start 150.823038 78.953145) (end 147.082038 82.694145) (width 0.2) (layer "B.Cu") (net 6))
 (segment (start 177.196288 65.113835) (end 177.196288 72.111145) (width 0.2) (layer "F.Cu") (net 7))
 (segment (start 171.734538 82.694145) (end 172.114538 82.314145) (width 0.2) (layer "F.Cu") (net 7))
 (segment (start 166.132038 63.644145) (end 166.979038 64.491145) (width 0.2) (layer "F.Cu") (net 7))
 (segment (start 176.573598 64.491145) (end 177.196288 65.113835) (width 0.2) (layer "F.Cu") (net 7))
 (segment (start 166.132038 82.694145) (end 171.734538 82.694145) (width 0.2) (layer "F.Cu") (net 7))
 (segment (start 177.196288 72.111145) (end 176.133288 73.174145) (width 0.2) (layer "F.Cu") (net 7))
 (segment (start 166.979038 64.491145) (end 176.573598 64.491145) (width 0.2) (layer "F.Cu") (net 7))
 (via (at 172.114538 82.314145) (size 0.6) (drill 0.3) (layers "F.Cu" "B.Cu") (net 7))
 (segment (start 166.767038 82.694145) (end 166.132038 82.694145) (width 0.2) (layer "B.Cu") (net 7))
 (segment (start 174.964538 73.174145) (end 176.133288 73.174145) (width 0.2) (layer "B.Cu") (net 7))
 (segment (start 172.114538 82.314145) (end 172.114538 76.024145) (width 0.2) (layer "B.Cu") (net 7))
 (segment (start 172.114538 76.024145) (end 174.964538 73.174145) (width 0.2) (layer "B.Cu") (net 7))
 (segment (start 117.584709 95.592) (end 106.002709 84.01) (width 0.2) (layer "F.Cu") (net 1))
 (segment (start 176.668 95.592) (end 117.584709 95.592) (width 0.2) (layer "F.Cu") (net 1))
 (segment (start 182.5 89.76) (end 176.668 95.592) (width 0.2) (layer "F.Cu") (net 1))
 (segment (start 106.002709 84.01) (end 103.856183 84.01) (width 0.2) (layer "F.Cu") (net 1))
 (segment (start 103.856183 84.01) (end 102.632038 85.234145) (width 0.2) (layer "F.Cu") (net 1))
 (segment (start 185.17 97.02) (end 127.43 97.02) (width 0.2) (layer "F.Cu") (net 19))
 (segment (start 192.43 89.76) (end 185.17 97.02) (width 0.2) (layer "F.Cu") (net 19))
 (via (at 127.43 97.02) (size 0.6) (drill 0.3) (layers "F.Cu" "B.Cu") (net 19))
 (segment (start 121.682038 91.272038) (end 121.682038 85.234145) (width 0.2) (layer "B.Cu") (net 19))
 (segment (start 127.43 97.02) (end 121.682038 91.272038) (width 0.2) (layer "B.Cu") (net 19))
 (segment (start 180.33 96.29) (end 139.78 96.29) (width 0.2) (layer "F.Cu") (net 16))
 (segment (start 182.53 94.09) (end 180.33 96.29) (width 0.2) (layer "F.Cu") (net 16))
 (via (at 139.78 96.29) (size 0.6) (drill 0.3) (layers "F.Cu" "B.Cu") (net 16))
 (segment (start 139.78 96.29) (end 140.732038 95.337962) (width 0.2) (layer "B.Cu") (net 16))
 (segment (start 140.732038 95.337962) (end 140.732038 85.234145) (width 0.2) (layer "B.Cu") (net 16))
 (segment (start 101.231038 66.894675) (end 108.982038 74.645675) (width 0.2) (layer "F.Cu") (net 4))
 (segment (start 108.982038 74.645675) (end 108.982038 82.694145) (width 0.2) (layer "F.Cu") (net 4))
 (segment (start 127.800724 65.394145) (end 139.540724 65.394145) (width 0.2) (layer "F.Cu") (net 4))
 (segment (start 108.982038 63.644145) (end 103.190724 63.644145) (width 0.2) (layer "F.Cu") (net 4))
 (segment (start 139.540724 65.394145) (end 140.151724 64.783145) (width 0.2) (layer "F.Cu") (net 4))
 (segment (start 165.289724 64.783145) (end 166.060724 65.554145) (width 0.2) (layer "F.Cu") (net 4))
 (segment (start 148.181724 64.783145) (end 165.289724 64.783145) (width 0.2) (layer "F.Cu") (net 4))
 (segment (start 147.210724 65.754145) (end 148.181724 64.783145) (width 0.2) (layer "F.Cu") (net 4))
 (segment (start 140.151724 64.783145) (end 146.239724 64.783145) (width 0.2) (layer "F.Cu") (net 4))
 (segment (start 103.190724 63.644145) (end 101.231038 65.603831) (width 0.2) (layer "F.Cu") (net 4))
 (segment (start 146.239724 64.783145) (end 147.210724 65.754145) (width 0.2) (layer "F.Cu") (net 4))
 (segment (start 101.231038 65.603831) (end 101.231038 66.894675) (width 0.2) (layer "F.Cu") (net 4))
 (segment (start 166.060724 65.554145) (end 176.133288 65.554145) (width 0.2) (layer "F.Cu") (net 4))
 (segment (start 126.050724 63.644145) (end 127.800724 65.394145) (width 0.2) (layer "F.Cu") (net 4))
 (segment (start 108.982038 63.644145) (end 126.050724 63.644145) (width 0.2) (layer "F.Cu") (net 4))
 (segment (start 175.69516 95.191) (end 174.12484 95.191) (width 0.2) (layer "F.Cu") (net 22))
 (segment (start 178.823538 85.08693) (end 178.823538 92.062622) (width 0.2) (layer "F.Cu") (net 22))
 (segment (start 107.226854 66.184145) (end 102.632038 66.184145) (width 0.2) (layer "F.Cu") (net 22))
 (segment (start 174.12484 95.191) (end 173.669 94.73516) (width 0.2) (layer "F.Cu") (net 22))
 (segment (start 173.669 94.73516) (end 173.669 82.693023) (width 0.2) (layer "F.Cu") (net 22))
 (segment (start 171.311122 80.335145) (end 121.377854 80.335145) (width 0.2) (layer "F.Cu") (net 22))
 (segment (start 182.4039 81.506568) (end 178.823538 85.08693) (width 0.2) (layer "F.Cu") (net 22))
 (segment (start 121.377854 80.335145) (end 107.226854 66.184145) (width 0.2) (layer "F.Cu") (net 22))
 (segment (start 178.823538 92.062622) (end 175.69516 95.191) (width 0.2) (layer "F.Cu") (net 22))
 (segment (start 173.669 82.693023) (end 171.311122 80.335145) (width 0.2) (layer "F.Cu") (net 22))
 (segment (start 102.585788 66.230395) (end 102.632038 66.184145) (width 0.2) (layer "F.Cu") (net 22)))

